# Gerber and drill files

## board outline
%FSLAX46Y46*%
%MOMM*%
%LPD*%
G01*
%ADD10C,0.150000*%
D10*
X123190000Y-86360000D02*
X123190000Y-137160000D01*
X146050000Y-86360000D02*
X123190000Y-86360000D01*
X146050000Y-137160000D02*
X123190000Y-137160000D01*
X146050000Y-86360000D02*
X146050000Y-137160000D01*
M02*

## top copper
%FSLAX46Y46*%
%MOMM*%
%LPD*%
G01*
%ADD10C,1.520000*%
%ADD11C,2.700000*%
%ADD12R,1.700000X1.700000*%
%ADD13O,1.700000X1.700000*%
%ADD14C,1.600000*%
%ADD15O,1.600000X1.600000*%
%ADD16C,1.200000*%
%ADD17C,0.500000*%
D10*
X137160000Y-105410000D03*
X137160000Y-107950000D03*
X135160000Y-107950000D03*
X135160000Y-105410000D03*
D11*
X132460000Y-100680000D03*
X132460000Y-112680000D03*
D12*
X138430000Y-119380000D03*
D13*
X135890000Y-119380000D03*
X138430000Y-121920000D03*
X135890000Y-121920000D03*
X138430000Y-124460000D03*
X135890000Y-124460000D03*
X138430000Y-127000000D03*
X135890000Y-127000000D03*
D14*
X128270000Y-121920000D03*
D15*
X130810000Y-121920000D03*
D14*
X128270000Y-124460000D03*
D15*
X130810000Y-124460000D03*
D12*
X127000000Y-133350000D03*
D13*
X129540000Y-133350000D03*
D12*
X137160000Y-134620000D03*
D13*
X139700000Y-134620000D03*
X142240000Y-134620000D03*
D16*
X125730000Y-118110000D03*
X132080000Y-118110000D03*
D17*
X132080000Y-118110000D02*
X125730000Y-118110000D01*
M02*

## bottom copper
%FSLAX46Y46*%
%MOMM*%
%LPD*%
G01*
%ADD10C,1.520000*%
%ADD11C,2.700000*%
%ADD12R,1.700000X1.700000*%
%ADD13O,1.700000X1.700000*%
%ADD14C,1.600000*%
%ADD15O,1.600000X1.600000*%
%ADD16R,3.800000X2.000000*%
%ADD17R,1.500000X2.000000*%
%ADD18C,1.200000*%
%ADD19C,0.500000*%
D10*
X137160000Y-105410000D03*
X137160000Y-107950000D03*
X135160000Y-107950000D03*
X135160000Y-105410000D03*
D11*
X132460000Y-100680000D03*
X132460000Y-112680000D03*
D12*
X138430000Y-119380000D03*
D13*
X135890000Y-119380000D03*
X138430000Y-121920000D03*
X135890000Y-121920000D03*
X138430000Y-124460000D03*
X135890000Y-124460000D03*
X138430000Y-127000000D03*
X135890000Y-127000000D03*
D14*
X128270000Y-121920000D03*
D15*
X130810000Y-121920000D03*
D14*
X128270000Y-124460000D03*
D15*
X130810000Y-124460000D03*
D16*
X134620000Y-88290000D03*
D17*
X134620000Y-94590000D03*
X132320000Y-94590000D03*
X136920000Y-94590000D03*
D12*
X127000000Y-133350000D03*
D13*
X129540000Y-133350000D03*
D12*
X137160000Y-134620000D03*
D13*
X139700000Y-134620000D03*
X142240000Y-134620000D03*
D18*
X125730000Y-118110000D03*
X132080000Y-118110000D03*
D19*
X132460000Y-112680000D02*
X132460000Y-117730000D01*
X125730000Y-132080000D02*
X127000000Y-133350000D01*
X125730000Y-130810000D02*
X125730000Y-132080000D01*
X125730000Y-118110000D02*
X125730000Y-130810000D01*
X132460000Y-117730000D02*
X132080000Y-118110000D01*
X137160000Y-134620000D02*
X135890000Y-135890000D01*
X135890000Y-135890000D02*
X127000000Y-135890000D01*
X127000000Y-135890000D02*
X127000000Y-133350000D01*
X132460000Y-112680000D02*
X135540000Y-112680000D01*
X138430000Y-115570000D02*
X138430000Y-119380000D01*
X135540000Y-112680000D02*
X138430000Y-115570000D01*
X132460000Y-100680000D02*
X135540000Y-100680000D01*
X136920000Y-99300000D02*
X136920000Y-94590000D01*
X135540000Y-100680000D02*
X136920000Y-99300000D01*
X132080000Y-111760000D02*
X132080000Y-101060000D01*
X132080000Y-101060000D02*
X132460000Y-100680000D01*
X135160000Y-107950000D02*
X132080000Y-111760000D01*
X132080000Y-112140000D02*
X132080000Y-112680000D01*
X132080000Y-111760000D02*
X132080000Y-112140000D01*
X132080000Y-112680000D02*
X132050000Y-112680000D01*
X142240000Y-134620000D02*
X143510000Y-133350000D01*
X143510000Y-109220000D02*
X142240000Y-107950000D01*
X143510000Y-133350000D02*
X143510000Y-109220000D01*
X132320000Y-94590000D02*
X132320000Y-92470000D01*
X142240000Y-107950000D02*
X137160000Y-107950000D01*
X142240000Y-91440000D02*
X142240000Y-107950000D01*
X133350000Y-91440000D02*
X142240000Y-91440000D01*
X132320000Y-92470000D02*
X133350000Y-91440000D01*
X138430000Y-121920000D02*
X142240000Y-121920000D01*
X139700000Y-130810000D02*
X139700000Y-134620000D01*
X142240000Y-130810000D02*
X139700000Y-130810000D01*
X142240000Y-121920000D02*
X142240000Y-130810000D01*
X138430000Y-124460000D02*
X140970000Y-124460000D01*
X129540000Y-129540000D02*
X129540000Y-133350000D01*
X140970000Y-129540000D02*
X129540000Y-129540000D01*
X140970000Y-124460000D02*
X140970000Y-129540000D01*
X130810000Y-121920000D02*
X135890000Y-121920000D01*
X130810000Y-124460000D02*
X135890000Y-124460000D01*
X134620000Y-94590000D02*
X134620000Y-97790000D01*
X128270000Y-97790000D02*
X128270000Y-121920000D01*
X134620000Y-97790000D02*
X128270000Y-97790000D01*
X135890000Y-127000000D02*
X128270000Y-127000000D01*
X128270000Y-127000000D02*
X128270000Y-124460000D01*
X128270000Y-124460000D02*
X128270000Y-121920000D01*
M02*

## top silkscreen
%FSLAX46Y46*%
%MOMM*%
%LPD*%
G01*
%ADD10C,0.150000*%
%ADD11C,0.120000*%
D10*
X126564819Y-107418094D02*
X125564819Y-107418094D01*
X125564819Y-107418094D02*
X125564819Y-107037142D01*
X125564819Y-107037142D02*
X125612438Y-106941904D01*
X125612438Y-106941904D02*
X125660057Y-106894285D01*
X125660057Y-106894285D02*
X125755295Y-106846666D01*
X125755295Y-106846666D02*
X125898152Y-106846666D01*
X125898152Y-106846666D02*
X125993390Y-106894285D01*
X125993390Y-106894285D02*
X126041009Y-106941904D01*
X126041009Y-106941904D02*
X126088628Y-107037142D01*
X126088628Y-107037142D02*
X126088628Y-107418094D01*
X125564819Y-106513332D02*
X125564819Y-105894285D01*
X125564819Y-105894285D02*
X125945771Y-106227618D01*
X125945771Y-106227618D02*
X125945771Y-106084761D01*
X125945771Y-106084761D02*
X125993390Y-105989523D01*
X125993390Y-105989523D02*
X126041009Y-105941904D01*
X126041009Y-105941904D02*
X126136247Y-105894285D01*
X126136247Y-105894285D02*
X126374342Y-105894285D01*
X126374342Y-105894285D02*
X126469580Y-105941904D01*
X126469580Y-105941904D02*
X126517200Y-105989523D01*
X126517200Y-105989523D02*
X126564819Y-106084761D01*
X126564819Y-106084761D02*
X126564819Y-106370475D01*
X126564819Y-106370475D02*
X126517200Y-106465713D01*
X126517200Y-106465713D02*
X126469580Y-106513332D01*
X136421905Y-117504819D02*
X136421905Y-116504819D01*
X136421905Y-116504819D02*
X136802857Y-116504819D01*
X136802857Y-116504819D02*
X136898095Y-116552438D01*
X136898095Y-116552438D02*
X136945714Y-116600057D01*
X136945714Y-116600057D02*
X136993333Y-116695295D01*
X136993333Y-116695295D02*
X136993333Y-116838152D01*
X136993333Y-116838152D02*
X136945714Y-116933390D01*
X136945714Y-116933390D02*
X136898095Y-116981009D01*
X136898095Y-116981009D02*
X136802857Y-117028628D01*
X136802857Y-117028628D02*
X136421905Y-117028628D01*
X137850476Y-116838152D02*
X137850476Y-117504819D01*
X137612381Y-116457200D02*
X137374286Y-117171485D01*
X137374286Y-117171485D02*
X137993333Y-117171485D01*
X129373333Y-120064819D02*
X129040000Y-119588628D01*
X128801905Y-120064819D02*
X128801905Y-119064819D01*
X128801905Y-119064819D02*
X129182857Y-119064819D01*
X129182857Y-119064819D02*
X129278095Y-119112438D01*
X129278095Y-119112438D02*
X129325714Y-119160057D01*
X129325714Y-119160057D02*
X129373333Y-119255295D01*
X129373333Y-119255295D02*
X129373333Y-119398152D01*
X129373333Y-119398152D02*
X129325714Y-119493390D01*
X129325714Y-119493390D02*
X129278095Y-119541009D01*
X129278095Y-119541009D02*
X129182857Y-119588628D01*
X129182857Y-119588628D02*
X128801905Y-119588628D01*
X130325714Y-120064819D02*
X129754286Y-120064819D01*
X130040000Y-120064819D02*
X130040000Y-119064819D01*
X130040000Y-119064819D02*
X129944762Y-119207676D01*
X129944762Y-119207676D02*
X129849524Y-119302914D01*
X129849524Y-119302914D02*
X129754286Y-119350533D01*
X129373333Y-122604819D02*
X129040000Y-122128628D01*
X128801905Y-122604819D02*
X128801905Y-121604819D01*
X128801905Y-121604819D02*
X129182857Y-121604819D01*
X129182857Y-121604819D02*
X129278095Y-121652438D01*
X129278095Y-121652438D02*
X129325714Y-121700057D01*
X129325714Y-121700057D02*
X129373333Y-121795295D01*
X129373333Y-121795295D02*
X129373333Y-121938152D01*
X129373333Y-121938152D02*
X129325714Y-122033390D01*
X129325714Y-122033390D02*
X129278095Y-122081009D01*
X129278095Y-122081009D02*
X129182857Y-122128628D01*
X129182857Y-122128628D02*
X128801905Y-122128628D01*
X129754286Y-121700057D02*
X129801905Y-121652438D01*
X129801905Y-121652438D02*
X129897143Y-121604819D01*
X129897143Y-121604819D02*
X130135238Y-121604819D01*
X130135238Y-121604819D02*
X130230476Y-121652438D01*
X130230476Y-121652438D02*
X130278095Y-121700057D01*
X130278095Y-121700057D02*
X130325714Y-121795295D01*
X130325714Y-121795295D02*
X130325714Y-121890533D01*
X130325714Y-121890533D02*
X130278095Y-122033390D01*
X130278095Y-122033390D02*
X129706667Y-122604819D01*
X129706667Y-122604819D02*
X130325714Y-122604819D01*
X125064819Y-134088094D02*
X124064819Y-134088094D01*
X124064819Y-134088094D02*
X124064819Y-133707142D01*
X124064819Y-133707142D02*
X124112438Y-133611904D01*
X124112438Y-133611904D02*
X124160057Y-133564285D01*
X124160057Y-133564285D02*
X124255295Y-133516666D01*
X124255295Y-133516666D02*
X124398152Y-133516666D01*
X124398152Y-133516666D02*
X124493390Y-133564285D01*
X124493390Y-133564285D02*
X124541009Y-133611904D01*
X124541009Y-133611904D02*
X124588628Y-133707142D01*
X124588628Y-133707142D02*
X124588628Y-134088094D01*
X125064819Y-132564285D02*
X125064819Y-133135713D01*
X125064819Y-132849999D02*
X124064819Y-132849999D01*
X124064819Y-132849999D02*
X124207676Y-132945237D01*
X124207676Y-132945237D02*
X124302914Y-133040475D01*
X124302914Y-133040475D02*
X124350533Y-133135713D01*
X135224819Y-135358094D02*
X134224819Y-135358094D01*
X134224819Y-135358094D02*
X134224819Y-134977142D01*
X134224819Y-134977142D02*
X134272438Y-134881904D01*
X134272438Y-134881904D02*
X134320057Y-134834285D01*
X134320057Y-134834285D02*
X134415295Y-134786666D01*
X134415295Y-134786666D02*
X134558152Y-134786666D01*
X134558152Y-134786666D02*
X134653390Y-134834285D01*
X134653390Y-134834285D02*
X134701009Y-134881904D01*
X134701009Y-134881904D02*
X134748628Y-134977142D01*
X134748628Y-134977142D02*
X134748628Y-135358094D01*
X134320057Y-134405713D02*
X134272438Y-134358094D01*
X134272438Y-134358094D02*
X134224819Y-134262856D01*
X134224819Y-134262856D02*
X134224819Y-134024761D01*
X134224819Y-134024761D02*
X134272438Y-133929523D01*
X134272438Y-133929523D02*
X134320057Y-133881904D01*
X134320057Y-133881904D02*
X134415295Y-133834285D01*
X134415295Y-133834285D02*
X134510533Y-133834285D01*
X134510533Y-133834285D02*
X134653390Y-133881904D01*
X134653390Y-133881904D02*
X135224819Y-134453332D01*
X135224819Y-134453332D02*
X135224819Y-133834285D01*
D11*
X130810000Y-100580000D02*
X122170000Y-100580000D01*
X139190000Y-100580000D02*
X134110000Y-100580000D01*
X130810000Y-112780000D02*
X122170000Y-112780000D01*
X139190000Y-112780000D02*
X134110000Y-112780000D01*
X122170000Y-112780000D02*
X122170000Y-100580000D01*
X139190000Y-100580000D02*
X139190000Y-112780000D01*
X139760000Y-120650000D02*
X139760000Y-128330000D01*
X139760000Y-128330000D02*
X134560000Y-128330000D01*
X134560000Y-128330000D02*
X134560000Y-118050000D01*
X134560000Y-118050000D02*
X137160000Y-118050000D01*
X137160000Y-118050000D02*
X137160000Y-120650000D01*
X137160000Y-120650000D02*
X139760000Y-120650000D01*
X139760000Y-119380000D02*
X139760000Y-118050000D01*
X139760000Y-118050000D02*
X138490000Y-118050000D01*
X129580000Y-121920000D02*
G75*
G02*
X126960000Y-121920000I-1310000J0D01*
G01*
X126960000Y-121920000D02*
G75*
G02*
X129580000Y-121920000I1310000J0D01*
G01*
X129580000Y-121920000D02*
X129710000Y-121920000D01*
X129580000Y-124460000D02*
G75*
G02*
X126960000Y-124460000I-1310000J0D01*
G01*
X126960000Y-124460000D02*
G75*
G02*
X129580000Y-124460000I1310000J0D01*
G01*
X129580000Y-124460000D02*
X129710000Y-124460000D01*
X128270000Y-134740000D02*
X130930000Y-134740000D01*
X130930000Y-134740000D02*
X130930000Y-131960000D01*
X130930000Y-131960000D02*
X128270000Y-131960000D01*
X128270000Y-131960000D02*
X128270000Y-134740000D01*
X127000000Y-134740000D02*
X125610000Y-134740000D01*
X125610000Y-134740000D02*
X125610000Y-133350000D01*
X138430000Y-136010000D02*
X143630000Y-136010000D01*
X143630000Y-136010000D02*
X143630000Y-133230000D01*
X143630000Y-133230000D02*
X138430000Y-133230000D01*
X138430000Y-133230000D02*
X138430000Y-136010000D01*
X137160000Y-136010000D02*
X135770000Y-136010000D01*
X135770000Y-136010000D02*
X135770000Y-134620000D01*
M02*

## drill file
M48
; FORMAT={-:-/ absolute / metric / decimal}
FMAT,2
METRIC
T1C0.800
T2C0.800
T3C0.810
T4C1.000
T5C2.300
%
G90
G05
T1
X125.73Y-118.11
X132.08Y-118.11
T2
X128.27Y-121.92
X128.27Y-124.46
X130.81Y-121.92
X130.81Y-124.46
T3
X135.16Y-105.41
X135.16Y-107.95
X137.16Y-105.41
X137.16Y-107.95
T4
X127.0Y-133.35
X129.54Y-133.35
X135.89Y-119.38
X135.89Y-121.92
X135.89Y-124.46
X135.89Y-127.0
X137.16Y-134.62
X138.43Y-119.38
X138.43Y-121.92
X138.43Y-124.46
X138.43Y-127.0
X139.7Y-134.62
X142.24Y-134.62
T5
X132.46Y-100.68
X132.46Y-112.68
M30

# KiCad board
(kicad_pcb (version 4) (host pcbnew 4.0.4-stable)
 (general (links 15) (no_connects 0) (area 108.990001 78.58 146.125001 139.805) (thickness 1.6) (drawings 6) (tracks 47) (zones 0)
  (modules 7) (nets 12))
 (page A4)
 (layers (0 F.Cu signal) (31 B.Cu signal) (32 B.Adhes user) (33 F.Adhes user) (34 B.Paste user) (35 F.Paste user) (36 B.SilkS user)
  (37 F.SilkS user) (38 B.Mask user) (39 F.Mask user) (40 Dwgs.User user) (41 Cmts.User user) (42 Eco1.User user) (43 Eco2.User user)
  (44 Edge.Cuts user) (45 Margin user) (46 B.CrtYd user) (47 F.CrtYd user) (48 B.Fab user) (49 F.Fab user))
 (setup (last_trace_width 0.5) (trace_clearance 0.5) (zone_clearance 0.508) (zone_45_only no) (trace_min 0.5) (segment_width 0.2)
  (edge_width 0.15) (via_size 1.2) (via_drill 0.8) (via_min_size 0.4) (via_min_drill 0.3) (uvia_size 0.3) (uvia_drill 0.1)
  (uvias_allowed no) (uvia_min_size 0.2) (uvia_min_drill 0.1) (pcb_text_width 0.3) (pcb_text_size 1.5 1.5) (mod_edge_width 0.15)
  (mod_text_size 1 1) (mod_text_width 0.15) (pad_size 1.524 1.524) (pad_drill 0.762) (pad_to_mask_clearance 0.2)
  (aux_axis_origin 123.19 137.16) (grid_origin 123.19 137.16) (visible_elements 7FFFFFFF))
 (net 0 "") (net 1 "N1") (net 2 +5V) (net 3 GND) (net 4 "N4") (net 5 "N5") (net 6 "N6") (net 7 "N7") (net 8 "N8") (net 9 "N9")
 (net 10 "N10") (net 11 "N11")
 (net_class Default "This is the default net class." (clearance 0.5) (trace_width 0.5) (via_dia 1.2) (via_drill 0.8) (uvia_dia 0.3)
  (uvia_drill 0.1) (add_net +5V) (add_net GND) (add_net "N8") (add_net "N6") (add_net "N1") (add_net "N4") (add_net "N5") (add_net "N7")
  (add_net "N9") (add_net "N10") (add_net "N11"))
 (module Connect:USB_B (layer F.Cu) (at 137.16 107.95 180)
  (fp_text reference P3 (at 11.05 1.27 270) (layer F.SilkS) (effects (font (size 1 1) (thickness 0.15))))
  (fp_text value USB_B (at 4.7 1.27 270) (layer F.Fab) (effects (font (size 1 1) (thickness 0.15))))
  (fp_line (start 6.35 7.37) (end 14.99 7.37) (layer F.SilkS) (width 0.12))
  (fp_line (start -2.03 7.37) (end 3.05 7.37) (layer F.SilkS) (width 0.12))
  (fp_line (start 6.35 -4.83) (end 14.99 -4.83) (layer F.SilkS) (width 0.12))
  (fp_line (start -2.03 -4.83) (end 3.05 -4.83) (layer F.SilkS) (width 0.12))
  (fp_line (start 14.99 -4.83) (end 14.99 7.37) (layer F.SilkS) (width 0.12))
  (fp_line (start -2.03 7.37) (end -2.03 -4.83) (layer F.SilkS) (width 0.12))
  (pad 2 thru_hole circle (at 0 2.54 90) (size 1.52 1.52) (drill 0.81) (layers *.Cu *.Mask) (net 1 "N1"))
  (pad 1 thru_hole circle (at 0 0 90) (size 1.52 1.52) (drill 0.81) (layers *.Cu *.Mask) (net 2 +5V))
  (pad 4 thru_hole circle (at 2 0 90) (size 1.52 1.52) (drill 0.81) (layers *.Cu *.Mask) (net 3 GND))
  (pad 3 thru_hole circle (at 2 2.54 90) (size 1.52 1.52) (drill 0.81) (layers *.Cu *.Mask) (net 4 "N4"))
  (pad 5 thru_hole circle (at 4.7 7.27 90) (size 2.7 2.7) (drill 2.3) (layers *.Cu *.Mask) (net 3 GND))
  (pad 5 thru_hole circle (at 4.7 -4.73 90) (size 2.7 2.7) (drill 2.3) (layers *.Cu *.Mask) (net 3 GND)))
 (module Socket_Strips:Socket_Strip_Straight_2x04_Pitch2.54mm (layer F.Cu) (at 138.43 119.38)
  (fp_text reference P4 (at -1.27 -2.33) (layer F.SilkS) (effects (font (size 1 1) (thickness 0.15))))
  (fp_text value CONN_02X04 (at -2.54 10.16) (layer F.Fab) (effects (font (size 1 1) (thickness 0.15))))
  (fp_line (start 1.33 1.27) (end 1.33 8.95) (layer F.SilkS) (width 0.12))
  (fp_line (start 1.33 8.95) (end -3.87 8.95) (layer F.SilkS) (width 0.12))
  (fp_line (start -3.87 8.95) (end -3.87 -1.33) (layer F.SilkS) (width 0.12))
  (fp_line (start -3.87 -1.33) (end -1.27 -1.33) (layer F.SilkS) (width 0.12))
  (fp_line (start -1.27 -1.33) (end -1.27 1.27) (layer F.SilkS) (width 0.12))
  (fp_line (start -1.27 1.27) (end 1.33 1.27) (layer F.SilkS) (width 0.12))
  (fp_line (start 1.33 0) (end 1.33 -1.33) (layer F.SilkS) (width 0.12))
  (fp_line (start 1.33 -1.33) (end 0.06 -1.33) (layer F.SilkS) (width 0.12))
  (pad 1 thru_hole rect (at 0 0) (size 1.7 1.7) (drill 1) (layers *.Cu *.Mask) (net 3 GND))
  (pad 2 thru_hole oval (at -2.54 0) (size 1.7 1.7) (drill 1) (layers *.Cu *.Mask) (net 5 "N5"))
  (pad 3 thru_hole oval (at 0 2.54) (size 1.7 1.7) (drill 1) (layers *.Cu *.Mask) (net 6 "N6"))
  (pad 4 thru_hole oval (at -2.54 2.54) (size 1.7 1.7) (drill 1) (layers *.Cu *.Mask) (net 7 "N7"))
  (pad 5 thru_hole oval (at 0 5.08) (size 1.7 1.7) (drill 1) (layers *.Cu *.Mask) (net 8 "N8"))
  (pad 6 thru_hole oval (at -2.54 5.08) (size 1.7 1.7) (drill 1) (layers *.Cu *.Mask) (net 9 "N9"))
  (pad 7 thru_hole oval (at 0 7.62) (size 1.7 1.7) (drill 1) (layers *.Cu *.Mask) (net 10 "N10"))
  (pad 8 thru_hole oval (at -2.54 7.62) (size 1.7 1.7) (drill 1) (layers *.Cu *.Mask) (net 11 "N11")))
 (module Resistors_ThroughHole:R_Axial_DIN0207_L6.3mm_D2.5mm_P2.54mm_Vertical (layer F.Cu) (at 128.27 121.92)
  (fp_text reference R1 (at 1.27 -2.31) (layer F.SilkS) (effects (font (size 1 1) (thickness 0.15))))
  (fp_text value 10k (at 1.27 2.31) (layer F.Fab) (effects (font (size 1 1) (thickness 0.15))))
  (fp_circle (center 0 0) (end 1.31 0) (layer F.SilkS) (width 0.12))
  (fp_line (start 1.31 0) (end 1.44 0) (layer F.SilkS) (width 0.12))
  (pad 1 thru_hole circle (at 0 0) (size 1.6 1.6) (drill 0.8) (layers *.Cu *.Mask) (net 11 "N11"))
  (pad 2 thru_hole oval (at 2.54 0) (size 1.6 1.6) (drill 0.8) (layers *.Cu *.Mask) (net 7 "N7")))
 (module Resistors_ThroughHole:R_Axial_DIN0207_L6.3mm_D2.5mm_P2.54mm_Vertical (layer F.Cu) (at 128.27 124.46)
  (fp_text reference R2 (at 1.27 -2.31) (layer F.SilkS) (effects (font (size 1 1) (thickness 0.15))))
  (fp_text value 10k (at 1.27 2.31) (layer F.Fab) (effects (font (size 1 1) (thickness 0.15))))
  (fp_circle (center 0 0) (end 1.31 0) (layer F.SilkS) (width 0.12))
  (fp_line (start 1.31 0) (end 1.44 0) (layer F.SilkS) (width 0.12))
  (pad 1 thru_hole circle (at 0 0) (size 1.6 1.6) (drill 0.8) (layers *.Cu *.Mask) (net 11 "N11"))
  (pad 2 thru_hole oval (at 2.54 0) (size 1.6 1.6) (drill 0.8) (layers *.Cu *.Mask) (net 9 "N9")))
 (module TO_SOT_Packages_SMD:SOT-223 (layer B.Cu) (at 134.62 91.44 90)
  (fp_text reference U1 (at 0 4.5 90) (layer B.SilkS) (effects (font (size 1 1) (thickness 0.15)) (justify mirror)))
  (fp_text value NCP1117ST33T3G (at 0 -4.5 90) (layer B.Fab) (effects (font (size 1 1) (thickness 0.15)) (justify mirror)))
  (pad 4 smd rect (at 3.15 0 90) (size 2 3.8) (layers B.Cu B.Paste B.Mask))
  (pad 2 smd rect (at -3.15 0 90) (size 2 1.5) (layers B.Cu B.Paste B.Mask) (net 11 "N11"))
  (pad 3 smd rect (at -3.15 -2.3 90) (size 2 1.5) (layers B.Cu B.Paste B.Mask) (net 2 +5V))
  (pad 1 smd rect (at -3.15 2.3 90) (size 2 1.5) (layers B.Cu B.Paste B.Mask) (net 3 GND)))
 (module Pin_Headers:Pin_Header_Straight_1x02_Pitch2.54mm (layer F.Cu) (at 127 133.35 90)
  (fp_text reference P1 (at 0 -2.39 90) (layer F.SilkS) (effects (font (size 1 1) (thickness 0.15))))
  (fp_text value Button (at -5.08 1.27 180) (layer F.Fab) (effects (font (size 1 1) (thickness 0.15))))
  (fp_line (start -1.39 1.27) (end -1.39 3.93) (layer F.SilkS) (width 0.12))
  (fp_line (start -1.39 3.93) (end 1.39 3.93) (layer F.SilkS) (width 0.12))
  (fp_line (start 1.39 3.93) (end 1.39 1.27) (layer F.SilkS) (width 0.12))
  (fp_line (start 1.39 1.27) (end -1.39 1.27) (layer F.SilkS) (width 0.12))
  (fp_line (start -1.39 0) (end -1.39 -1.39) (layer F.SilkS) (width 0.12))
  (fp_line (start -1.39 -1.39) (end 0 -1.39) (layer F.SilkS) (width 0.12))
  (pad 1 thru_hole rect (at 0 0 90) (size 1.7 1.7) (drill 1) (layers *.Cu *.Mask) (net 3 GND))
  (pad 2 thru_hole oval (at 0 2.54 90) (size 1.7 1.7) (drill 1) (layers *.Cu *.Mask) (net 8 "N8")))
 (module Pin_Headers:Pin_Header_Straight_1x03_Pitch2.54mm (layer F.Cu) (at 137.16 134.62 90)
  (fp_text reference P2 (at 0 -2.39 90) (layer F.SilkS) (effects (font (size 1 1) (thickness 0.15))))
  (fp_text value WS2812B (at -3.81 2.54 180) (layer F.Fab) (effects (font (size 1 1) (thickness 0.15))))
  (fp_line (start -1.39 1.27) (end -1.39 6.47) (layer F.SilkS) (width 0.12))
  (fp_line (start -1.39 6.47) (end 1.39 6.47) (layer F.SilkS) (width 0.12))
  (fp_line (start 1.39 6.47) (end 1.39 1.27) (layer F.SilkS) (width 0.12))
  (fp_line (start 1.39 1.27) (end -1.39 1.27) (layer F.SilkS) (width 0.12))
  (fp_line (start -1.39 0) (end -1.39 -1.39) (layer F.SilkS) (width 0.12))
  (fp_line (start -1.39 -1.39) (end 0 -1.39) (layer F.SilkS) (width 0.12))
  (pad 1 thru_hole rect (at 0 0 90) (size 1.7 1.7) (drill 1) (layers *.Cu *.Mask) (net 3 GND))
  (pad 2 thru_hole oval (at 0 2.54 90) (size 1.7 1.7) (drill 1) (layers *.Cu *.Mask) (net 6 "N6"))
  (pad 3 thru_hole oval (at 0 5.08 90) (size 1.7 1.7) (drill 1) (layers *.Cu *.Mask) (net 2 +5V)))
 (gr_line (start 123.19 86.36) (end 123.19 137.16) (angle 90) (layer Edge.Cuts) (width 0.15))
 (gr_line (start 146.05 86.36) (end 123.19 86.36) (angle 90) (layer Edge.Cuts) (width 0.15))
 (gr_line (start 146.05 137.16) (end 123.19 137.16) (angle 90) (layer Edge.Cuts) (width 0.15))
 (gr_line (start 146.05 86.36) (end 146.05 137.16) (angle 90) (layer Edge.Cuts) (width 0.15))
 (segment (start 132.46 112.68) (end 132.46 117.73) (width 0.5) (layer B.Cu) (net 3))
 (segment (start 125.73 132.08) (end 127 133.35) (width 0.5) (layer B.Cu) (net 3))
 (segment (start 125.73 130.81) (end 125.73 132.08) (width 0.5) (layer B.Cu) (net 3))
 (segment (start 125.73 118.11) (end 125.73 130.81) (width 0.5) (layer B.Cu) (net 3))
 (segment (start 132.08 118.11) (end 125.73 118.11) (width 0.5) (layer F.Cu) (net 3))
 (segment (start 132.46 117.73) (end 132.08 118.11) (width 0.5) (layer B.Cu) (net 3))
 (segment (start 137.16 134.62) (end 135.89 135.89) (width 0.5) (layer B.Cu) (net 3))
 (segment (start 135.89 135.89) (end 127 135.89) (width 0.5) (layer B.Cu) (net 3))
 (segment (start 127 135.89) (end 127 133.35) (width 0.5) (layer B.Cu) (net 3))
 (segment (start 132.46 112.68) (end 135.54 112.68) (width 0.5) (layer B.Cu) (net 3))
 (segment (start 138.43 115.57) (end 138.43 119.38) (width 0.5) (layer B.Cu) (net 3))
 (segment (start 135.54 112.68) (end 138.43 115.57) (width 0.5) (layer B.Cu) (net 3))
 (segment (start 132.46 100.68) (end 135.54 100.68) (width 0.5) (layer B.Cu) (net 3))
 (segment (start 136.92 99.3) (end 136.92 94.59) (width 0.5) (layer B.Cu) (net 3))
 (segment (start 135.54 100.68) (end 136.92 99.3) (width 0.5) (layer B.Cu) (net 3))
 (segment (start 132.08 111.76) (end 132.08 101.06) (width 0.5) (layer B.Cu) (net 3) (status 20))
 (segment (start 132.08 101.06) (end 132.46 100.68) (width 0.5) (layer B.Cu) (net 3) (status 30))
 (segment (start 135.16 107.95) (end 132.08 111.76) (width 0.5) (layer B.Cu) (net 3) (status 10))
 (segment (start 132.08 112.14) (end 132.08 112.68) (width 0.5) (layer B.Cu) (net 3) (status 20))
 (segment (start 132.08 111.76) (end 132.08 112.14) (width 0.5) (layer B.Cu) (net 3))
 (segment (start 132.08 112.68) (end 132.05 112.68) (width 0.5) (layer B.Cu) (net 3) (status 30))
 (segment (start 142.24 134.62) (end 143.51 133.35) (width 0.5) (layer B.Cu) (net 2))
 (segment (start 143.51 109.22) (end 142.24 107.95) (width 0.5) (layer B.Cu) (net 2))
 (segment (start 143.51 133.35) (end 143.51 109.22) (width 0.5) (layer B.Cu) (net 2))
 (segment (start 132.32 94.59) (end 132.32 92.47) (width 0.5) (layer B.Cu) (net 2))
 (segment (start 142.24 107.95) (end 137.16 107.95) (width 0.5) (layer B.Cu) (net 2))
 (segment (start 142.24 91.44) (end 142.24 107.95) (width 0.5) (layer B.Cu) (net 2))
 (segment (start 133.35 91.44) (end 142.24 91.44) (width 0.5) (layer B.Cu) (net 2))
 (segment (start 132.32 92.47) (end 133.35 91.44) (width 0.5) (layer B.Cu) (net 2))
 (segment (start 138.43 121.92) (end 142.24 121.92) (width 0.5) (layer B.Cu) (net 6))
 (segment (start 139.7 130.81) (end 139.7 134.62) (width 0.5) (layer B.Cu) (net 6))
 (segment (start 142.24 130.81) (end 139.7 130.81) (width 0.5) (layer B.Cu) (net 6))
 (segment (start 142.24 121.92) (end 142.24 130.81) (width 0.5) (layer B.Cu) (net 6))
 (segment (start 138.43 124.46) (end 140.97 124.46) (width 0.5) (layer B.Cu) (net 8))
 (segment (start 129.54 129.54) (end 129.54 133.35) (width 0.5) (layer B.Cu) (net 8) (status 20))
 (segment (start 140.97 129.54) (end 129.54 129.54) (width 0.5) (layer B.Cu) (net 8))
 (segment (start 140.97 124.46) (end 140.97 129.54) (width 0.5) (layer B.Cu) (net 8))
 (segment (start 130.81 121.92) (end 135.89 121.92) (width 0.5) (layer B.Cu) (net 7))
 (segment (start 130.81 124.46) (end 135.89 124.46) (width 0.5) (layer B.Cu) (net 9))
 (segment (start 134.62 94.59) (end 134.62 97.79) (width 0.5) (layer B.Cu) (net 11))
 (segment (start 128.27 97.79) (end 128.27 121.92) (width 0.5) (layer B.Cu) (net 11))
 (segment (start 134.62 97.79) (end 128.27 97.79) (width 0.5) (layer B.Cu) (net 11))
 (segment (start 135.89 127) (end 128.27 127) (width 0.5) (layer B.Cu) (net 11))
 (segment (start 128.27 127) (end 128.27 124.46) (width 0.5) (layer B.Cu) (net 11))
 (segment (start 128.27 124.46) (end 128.27 121.92) (width 0.5) (layer B.Cu) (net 11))
 (via (at 125.73 118.11) (size 1.2) (drill 0.8) (layers F.Cu B.Cu) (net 3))
 (via (at 132.08 118.11) (size 1.2) (drill 0.8) (layers F.Cu B.Cu) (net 3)))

